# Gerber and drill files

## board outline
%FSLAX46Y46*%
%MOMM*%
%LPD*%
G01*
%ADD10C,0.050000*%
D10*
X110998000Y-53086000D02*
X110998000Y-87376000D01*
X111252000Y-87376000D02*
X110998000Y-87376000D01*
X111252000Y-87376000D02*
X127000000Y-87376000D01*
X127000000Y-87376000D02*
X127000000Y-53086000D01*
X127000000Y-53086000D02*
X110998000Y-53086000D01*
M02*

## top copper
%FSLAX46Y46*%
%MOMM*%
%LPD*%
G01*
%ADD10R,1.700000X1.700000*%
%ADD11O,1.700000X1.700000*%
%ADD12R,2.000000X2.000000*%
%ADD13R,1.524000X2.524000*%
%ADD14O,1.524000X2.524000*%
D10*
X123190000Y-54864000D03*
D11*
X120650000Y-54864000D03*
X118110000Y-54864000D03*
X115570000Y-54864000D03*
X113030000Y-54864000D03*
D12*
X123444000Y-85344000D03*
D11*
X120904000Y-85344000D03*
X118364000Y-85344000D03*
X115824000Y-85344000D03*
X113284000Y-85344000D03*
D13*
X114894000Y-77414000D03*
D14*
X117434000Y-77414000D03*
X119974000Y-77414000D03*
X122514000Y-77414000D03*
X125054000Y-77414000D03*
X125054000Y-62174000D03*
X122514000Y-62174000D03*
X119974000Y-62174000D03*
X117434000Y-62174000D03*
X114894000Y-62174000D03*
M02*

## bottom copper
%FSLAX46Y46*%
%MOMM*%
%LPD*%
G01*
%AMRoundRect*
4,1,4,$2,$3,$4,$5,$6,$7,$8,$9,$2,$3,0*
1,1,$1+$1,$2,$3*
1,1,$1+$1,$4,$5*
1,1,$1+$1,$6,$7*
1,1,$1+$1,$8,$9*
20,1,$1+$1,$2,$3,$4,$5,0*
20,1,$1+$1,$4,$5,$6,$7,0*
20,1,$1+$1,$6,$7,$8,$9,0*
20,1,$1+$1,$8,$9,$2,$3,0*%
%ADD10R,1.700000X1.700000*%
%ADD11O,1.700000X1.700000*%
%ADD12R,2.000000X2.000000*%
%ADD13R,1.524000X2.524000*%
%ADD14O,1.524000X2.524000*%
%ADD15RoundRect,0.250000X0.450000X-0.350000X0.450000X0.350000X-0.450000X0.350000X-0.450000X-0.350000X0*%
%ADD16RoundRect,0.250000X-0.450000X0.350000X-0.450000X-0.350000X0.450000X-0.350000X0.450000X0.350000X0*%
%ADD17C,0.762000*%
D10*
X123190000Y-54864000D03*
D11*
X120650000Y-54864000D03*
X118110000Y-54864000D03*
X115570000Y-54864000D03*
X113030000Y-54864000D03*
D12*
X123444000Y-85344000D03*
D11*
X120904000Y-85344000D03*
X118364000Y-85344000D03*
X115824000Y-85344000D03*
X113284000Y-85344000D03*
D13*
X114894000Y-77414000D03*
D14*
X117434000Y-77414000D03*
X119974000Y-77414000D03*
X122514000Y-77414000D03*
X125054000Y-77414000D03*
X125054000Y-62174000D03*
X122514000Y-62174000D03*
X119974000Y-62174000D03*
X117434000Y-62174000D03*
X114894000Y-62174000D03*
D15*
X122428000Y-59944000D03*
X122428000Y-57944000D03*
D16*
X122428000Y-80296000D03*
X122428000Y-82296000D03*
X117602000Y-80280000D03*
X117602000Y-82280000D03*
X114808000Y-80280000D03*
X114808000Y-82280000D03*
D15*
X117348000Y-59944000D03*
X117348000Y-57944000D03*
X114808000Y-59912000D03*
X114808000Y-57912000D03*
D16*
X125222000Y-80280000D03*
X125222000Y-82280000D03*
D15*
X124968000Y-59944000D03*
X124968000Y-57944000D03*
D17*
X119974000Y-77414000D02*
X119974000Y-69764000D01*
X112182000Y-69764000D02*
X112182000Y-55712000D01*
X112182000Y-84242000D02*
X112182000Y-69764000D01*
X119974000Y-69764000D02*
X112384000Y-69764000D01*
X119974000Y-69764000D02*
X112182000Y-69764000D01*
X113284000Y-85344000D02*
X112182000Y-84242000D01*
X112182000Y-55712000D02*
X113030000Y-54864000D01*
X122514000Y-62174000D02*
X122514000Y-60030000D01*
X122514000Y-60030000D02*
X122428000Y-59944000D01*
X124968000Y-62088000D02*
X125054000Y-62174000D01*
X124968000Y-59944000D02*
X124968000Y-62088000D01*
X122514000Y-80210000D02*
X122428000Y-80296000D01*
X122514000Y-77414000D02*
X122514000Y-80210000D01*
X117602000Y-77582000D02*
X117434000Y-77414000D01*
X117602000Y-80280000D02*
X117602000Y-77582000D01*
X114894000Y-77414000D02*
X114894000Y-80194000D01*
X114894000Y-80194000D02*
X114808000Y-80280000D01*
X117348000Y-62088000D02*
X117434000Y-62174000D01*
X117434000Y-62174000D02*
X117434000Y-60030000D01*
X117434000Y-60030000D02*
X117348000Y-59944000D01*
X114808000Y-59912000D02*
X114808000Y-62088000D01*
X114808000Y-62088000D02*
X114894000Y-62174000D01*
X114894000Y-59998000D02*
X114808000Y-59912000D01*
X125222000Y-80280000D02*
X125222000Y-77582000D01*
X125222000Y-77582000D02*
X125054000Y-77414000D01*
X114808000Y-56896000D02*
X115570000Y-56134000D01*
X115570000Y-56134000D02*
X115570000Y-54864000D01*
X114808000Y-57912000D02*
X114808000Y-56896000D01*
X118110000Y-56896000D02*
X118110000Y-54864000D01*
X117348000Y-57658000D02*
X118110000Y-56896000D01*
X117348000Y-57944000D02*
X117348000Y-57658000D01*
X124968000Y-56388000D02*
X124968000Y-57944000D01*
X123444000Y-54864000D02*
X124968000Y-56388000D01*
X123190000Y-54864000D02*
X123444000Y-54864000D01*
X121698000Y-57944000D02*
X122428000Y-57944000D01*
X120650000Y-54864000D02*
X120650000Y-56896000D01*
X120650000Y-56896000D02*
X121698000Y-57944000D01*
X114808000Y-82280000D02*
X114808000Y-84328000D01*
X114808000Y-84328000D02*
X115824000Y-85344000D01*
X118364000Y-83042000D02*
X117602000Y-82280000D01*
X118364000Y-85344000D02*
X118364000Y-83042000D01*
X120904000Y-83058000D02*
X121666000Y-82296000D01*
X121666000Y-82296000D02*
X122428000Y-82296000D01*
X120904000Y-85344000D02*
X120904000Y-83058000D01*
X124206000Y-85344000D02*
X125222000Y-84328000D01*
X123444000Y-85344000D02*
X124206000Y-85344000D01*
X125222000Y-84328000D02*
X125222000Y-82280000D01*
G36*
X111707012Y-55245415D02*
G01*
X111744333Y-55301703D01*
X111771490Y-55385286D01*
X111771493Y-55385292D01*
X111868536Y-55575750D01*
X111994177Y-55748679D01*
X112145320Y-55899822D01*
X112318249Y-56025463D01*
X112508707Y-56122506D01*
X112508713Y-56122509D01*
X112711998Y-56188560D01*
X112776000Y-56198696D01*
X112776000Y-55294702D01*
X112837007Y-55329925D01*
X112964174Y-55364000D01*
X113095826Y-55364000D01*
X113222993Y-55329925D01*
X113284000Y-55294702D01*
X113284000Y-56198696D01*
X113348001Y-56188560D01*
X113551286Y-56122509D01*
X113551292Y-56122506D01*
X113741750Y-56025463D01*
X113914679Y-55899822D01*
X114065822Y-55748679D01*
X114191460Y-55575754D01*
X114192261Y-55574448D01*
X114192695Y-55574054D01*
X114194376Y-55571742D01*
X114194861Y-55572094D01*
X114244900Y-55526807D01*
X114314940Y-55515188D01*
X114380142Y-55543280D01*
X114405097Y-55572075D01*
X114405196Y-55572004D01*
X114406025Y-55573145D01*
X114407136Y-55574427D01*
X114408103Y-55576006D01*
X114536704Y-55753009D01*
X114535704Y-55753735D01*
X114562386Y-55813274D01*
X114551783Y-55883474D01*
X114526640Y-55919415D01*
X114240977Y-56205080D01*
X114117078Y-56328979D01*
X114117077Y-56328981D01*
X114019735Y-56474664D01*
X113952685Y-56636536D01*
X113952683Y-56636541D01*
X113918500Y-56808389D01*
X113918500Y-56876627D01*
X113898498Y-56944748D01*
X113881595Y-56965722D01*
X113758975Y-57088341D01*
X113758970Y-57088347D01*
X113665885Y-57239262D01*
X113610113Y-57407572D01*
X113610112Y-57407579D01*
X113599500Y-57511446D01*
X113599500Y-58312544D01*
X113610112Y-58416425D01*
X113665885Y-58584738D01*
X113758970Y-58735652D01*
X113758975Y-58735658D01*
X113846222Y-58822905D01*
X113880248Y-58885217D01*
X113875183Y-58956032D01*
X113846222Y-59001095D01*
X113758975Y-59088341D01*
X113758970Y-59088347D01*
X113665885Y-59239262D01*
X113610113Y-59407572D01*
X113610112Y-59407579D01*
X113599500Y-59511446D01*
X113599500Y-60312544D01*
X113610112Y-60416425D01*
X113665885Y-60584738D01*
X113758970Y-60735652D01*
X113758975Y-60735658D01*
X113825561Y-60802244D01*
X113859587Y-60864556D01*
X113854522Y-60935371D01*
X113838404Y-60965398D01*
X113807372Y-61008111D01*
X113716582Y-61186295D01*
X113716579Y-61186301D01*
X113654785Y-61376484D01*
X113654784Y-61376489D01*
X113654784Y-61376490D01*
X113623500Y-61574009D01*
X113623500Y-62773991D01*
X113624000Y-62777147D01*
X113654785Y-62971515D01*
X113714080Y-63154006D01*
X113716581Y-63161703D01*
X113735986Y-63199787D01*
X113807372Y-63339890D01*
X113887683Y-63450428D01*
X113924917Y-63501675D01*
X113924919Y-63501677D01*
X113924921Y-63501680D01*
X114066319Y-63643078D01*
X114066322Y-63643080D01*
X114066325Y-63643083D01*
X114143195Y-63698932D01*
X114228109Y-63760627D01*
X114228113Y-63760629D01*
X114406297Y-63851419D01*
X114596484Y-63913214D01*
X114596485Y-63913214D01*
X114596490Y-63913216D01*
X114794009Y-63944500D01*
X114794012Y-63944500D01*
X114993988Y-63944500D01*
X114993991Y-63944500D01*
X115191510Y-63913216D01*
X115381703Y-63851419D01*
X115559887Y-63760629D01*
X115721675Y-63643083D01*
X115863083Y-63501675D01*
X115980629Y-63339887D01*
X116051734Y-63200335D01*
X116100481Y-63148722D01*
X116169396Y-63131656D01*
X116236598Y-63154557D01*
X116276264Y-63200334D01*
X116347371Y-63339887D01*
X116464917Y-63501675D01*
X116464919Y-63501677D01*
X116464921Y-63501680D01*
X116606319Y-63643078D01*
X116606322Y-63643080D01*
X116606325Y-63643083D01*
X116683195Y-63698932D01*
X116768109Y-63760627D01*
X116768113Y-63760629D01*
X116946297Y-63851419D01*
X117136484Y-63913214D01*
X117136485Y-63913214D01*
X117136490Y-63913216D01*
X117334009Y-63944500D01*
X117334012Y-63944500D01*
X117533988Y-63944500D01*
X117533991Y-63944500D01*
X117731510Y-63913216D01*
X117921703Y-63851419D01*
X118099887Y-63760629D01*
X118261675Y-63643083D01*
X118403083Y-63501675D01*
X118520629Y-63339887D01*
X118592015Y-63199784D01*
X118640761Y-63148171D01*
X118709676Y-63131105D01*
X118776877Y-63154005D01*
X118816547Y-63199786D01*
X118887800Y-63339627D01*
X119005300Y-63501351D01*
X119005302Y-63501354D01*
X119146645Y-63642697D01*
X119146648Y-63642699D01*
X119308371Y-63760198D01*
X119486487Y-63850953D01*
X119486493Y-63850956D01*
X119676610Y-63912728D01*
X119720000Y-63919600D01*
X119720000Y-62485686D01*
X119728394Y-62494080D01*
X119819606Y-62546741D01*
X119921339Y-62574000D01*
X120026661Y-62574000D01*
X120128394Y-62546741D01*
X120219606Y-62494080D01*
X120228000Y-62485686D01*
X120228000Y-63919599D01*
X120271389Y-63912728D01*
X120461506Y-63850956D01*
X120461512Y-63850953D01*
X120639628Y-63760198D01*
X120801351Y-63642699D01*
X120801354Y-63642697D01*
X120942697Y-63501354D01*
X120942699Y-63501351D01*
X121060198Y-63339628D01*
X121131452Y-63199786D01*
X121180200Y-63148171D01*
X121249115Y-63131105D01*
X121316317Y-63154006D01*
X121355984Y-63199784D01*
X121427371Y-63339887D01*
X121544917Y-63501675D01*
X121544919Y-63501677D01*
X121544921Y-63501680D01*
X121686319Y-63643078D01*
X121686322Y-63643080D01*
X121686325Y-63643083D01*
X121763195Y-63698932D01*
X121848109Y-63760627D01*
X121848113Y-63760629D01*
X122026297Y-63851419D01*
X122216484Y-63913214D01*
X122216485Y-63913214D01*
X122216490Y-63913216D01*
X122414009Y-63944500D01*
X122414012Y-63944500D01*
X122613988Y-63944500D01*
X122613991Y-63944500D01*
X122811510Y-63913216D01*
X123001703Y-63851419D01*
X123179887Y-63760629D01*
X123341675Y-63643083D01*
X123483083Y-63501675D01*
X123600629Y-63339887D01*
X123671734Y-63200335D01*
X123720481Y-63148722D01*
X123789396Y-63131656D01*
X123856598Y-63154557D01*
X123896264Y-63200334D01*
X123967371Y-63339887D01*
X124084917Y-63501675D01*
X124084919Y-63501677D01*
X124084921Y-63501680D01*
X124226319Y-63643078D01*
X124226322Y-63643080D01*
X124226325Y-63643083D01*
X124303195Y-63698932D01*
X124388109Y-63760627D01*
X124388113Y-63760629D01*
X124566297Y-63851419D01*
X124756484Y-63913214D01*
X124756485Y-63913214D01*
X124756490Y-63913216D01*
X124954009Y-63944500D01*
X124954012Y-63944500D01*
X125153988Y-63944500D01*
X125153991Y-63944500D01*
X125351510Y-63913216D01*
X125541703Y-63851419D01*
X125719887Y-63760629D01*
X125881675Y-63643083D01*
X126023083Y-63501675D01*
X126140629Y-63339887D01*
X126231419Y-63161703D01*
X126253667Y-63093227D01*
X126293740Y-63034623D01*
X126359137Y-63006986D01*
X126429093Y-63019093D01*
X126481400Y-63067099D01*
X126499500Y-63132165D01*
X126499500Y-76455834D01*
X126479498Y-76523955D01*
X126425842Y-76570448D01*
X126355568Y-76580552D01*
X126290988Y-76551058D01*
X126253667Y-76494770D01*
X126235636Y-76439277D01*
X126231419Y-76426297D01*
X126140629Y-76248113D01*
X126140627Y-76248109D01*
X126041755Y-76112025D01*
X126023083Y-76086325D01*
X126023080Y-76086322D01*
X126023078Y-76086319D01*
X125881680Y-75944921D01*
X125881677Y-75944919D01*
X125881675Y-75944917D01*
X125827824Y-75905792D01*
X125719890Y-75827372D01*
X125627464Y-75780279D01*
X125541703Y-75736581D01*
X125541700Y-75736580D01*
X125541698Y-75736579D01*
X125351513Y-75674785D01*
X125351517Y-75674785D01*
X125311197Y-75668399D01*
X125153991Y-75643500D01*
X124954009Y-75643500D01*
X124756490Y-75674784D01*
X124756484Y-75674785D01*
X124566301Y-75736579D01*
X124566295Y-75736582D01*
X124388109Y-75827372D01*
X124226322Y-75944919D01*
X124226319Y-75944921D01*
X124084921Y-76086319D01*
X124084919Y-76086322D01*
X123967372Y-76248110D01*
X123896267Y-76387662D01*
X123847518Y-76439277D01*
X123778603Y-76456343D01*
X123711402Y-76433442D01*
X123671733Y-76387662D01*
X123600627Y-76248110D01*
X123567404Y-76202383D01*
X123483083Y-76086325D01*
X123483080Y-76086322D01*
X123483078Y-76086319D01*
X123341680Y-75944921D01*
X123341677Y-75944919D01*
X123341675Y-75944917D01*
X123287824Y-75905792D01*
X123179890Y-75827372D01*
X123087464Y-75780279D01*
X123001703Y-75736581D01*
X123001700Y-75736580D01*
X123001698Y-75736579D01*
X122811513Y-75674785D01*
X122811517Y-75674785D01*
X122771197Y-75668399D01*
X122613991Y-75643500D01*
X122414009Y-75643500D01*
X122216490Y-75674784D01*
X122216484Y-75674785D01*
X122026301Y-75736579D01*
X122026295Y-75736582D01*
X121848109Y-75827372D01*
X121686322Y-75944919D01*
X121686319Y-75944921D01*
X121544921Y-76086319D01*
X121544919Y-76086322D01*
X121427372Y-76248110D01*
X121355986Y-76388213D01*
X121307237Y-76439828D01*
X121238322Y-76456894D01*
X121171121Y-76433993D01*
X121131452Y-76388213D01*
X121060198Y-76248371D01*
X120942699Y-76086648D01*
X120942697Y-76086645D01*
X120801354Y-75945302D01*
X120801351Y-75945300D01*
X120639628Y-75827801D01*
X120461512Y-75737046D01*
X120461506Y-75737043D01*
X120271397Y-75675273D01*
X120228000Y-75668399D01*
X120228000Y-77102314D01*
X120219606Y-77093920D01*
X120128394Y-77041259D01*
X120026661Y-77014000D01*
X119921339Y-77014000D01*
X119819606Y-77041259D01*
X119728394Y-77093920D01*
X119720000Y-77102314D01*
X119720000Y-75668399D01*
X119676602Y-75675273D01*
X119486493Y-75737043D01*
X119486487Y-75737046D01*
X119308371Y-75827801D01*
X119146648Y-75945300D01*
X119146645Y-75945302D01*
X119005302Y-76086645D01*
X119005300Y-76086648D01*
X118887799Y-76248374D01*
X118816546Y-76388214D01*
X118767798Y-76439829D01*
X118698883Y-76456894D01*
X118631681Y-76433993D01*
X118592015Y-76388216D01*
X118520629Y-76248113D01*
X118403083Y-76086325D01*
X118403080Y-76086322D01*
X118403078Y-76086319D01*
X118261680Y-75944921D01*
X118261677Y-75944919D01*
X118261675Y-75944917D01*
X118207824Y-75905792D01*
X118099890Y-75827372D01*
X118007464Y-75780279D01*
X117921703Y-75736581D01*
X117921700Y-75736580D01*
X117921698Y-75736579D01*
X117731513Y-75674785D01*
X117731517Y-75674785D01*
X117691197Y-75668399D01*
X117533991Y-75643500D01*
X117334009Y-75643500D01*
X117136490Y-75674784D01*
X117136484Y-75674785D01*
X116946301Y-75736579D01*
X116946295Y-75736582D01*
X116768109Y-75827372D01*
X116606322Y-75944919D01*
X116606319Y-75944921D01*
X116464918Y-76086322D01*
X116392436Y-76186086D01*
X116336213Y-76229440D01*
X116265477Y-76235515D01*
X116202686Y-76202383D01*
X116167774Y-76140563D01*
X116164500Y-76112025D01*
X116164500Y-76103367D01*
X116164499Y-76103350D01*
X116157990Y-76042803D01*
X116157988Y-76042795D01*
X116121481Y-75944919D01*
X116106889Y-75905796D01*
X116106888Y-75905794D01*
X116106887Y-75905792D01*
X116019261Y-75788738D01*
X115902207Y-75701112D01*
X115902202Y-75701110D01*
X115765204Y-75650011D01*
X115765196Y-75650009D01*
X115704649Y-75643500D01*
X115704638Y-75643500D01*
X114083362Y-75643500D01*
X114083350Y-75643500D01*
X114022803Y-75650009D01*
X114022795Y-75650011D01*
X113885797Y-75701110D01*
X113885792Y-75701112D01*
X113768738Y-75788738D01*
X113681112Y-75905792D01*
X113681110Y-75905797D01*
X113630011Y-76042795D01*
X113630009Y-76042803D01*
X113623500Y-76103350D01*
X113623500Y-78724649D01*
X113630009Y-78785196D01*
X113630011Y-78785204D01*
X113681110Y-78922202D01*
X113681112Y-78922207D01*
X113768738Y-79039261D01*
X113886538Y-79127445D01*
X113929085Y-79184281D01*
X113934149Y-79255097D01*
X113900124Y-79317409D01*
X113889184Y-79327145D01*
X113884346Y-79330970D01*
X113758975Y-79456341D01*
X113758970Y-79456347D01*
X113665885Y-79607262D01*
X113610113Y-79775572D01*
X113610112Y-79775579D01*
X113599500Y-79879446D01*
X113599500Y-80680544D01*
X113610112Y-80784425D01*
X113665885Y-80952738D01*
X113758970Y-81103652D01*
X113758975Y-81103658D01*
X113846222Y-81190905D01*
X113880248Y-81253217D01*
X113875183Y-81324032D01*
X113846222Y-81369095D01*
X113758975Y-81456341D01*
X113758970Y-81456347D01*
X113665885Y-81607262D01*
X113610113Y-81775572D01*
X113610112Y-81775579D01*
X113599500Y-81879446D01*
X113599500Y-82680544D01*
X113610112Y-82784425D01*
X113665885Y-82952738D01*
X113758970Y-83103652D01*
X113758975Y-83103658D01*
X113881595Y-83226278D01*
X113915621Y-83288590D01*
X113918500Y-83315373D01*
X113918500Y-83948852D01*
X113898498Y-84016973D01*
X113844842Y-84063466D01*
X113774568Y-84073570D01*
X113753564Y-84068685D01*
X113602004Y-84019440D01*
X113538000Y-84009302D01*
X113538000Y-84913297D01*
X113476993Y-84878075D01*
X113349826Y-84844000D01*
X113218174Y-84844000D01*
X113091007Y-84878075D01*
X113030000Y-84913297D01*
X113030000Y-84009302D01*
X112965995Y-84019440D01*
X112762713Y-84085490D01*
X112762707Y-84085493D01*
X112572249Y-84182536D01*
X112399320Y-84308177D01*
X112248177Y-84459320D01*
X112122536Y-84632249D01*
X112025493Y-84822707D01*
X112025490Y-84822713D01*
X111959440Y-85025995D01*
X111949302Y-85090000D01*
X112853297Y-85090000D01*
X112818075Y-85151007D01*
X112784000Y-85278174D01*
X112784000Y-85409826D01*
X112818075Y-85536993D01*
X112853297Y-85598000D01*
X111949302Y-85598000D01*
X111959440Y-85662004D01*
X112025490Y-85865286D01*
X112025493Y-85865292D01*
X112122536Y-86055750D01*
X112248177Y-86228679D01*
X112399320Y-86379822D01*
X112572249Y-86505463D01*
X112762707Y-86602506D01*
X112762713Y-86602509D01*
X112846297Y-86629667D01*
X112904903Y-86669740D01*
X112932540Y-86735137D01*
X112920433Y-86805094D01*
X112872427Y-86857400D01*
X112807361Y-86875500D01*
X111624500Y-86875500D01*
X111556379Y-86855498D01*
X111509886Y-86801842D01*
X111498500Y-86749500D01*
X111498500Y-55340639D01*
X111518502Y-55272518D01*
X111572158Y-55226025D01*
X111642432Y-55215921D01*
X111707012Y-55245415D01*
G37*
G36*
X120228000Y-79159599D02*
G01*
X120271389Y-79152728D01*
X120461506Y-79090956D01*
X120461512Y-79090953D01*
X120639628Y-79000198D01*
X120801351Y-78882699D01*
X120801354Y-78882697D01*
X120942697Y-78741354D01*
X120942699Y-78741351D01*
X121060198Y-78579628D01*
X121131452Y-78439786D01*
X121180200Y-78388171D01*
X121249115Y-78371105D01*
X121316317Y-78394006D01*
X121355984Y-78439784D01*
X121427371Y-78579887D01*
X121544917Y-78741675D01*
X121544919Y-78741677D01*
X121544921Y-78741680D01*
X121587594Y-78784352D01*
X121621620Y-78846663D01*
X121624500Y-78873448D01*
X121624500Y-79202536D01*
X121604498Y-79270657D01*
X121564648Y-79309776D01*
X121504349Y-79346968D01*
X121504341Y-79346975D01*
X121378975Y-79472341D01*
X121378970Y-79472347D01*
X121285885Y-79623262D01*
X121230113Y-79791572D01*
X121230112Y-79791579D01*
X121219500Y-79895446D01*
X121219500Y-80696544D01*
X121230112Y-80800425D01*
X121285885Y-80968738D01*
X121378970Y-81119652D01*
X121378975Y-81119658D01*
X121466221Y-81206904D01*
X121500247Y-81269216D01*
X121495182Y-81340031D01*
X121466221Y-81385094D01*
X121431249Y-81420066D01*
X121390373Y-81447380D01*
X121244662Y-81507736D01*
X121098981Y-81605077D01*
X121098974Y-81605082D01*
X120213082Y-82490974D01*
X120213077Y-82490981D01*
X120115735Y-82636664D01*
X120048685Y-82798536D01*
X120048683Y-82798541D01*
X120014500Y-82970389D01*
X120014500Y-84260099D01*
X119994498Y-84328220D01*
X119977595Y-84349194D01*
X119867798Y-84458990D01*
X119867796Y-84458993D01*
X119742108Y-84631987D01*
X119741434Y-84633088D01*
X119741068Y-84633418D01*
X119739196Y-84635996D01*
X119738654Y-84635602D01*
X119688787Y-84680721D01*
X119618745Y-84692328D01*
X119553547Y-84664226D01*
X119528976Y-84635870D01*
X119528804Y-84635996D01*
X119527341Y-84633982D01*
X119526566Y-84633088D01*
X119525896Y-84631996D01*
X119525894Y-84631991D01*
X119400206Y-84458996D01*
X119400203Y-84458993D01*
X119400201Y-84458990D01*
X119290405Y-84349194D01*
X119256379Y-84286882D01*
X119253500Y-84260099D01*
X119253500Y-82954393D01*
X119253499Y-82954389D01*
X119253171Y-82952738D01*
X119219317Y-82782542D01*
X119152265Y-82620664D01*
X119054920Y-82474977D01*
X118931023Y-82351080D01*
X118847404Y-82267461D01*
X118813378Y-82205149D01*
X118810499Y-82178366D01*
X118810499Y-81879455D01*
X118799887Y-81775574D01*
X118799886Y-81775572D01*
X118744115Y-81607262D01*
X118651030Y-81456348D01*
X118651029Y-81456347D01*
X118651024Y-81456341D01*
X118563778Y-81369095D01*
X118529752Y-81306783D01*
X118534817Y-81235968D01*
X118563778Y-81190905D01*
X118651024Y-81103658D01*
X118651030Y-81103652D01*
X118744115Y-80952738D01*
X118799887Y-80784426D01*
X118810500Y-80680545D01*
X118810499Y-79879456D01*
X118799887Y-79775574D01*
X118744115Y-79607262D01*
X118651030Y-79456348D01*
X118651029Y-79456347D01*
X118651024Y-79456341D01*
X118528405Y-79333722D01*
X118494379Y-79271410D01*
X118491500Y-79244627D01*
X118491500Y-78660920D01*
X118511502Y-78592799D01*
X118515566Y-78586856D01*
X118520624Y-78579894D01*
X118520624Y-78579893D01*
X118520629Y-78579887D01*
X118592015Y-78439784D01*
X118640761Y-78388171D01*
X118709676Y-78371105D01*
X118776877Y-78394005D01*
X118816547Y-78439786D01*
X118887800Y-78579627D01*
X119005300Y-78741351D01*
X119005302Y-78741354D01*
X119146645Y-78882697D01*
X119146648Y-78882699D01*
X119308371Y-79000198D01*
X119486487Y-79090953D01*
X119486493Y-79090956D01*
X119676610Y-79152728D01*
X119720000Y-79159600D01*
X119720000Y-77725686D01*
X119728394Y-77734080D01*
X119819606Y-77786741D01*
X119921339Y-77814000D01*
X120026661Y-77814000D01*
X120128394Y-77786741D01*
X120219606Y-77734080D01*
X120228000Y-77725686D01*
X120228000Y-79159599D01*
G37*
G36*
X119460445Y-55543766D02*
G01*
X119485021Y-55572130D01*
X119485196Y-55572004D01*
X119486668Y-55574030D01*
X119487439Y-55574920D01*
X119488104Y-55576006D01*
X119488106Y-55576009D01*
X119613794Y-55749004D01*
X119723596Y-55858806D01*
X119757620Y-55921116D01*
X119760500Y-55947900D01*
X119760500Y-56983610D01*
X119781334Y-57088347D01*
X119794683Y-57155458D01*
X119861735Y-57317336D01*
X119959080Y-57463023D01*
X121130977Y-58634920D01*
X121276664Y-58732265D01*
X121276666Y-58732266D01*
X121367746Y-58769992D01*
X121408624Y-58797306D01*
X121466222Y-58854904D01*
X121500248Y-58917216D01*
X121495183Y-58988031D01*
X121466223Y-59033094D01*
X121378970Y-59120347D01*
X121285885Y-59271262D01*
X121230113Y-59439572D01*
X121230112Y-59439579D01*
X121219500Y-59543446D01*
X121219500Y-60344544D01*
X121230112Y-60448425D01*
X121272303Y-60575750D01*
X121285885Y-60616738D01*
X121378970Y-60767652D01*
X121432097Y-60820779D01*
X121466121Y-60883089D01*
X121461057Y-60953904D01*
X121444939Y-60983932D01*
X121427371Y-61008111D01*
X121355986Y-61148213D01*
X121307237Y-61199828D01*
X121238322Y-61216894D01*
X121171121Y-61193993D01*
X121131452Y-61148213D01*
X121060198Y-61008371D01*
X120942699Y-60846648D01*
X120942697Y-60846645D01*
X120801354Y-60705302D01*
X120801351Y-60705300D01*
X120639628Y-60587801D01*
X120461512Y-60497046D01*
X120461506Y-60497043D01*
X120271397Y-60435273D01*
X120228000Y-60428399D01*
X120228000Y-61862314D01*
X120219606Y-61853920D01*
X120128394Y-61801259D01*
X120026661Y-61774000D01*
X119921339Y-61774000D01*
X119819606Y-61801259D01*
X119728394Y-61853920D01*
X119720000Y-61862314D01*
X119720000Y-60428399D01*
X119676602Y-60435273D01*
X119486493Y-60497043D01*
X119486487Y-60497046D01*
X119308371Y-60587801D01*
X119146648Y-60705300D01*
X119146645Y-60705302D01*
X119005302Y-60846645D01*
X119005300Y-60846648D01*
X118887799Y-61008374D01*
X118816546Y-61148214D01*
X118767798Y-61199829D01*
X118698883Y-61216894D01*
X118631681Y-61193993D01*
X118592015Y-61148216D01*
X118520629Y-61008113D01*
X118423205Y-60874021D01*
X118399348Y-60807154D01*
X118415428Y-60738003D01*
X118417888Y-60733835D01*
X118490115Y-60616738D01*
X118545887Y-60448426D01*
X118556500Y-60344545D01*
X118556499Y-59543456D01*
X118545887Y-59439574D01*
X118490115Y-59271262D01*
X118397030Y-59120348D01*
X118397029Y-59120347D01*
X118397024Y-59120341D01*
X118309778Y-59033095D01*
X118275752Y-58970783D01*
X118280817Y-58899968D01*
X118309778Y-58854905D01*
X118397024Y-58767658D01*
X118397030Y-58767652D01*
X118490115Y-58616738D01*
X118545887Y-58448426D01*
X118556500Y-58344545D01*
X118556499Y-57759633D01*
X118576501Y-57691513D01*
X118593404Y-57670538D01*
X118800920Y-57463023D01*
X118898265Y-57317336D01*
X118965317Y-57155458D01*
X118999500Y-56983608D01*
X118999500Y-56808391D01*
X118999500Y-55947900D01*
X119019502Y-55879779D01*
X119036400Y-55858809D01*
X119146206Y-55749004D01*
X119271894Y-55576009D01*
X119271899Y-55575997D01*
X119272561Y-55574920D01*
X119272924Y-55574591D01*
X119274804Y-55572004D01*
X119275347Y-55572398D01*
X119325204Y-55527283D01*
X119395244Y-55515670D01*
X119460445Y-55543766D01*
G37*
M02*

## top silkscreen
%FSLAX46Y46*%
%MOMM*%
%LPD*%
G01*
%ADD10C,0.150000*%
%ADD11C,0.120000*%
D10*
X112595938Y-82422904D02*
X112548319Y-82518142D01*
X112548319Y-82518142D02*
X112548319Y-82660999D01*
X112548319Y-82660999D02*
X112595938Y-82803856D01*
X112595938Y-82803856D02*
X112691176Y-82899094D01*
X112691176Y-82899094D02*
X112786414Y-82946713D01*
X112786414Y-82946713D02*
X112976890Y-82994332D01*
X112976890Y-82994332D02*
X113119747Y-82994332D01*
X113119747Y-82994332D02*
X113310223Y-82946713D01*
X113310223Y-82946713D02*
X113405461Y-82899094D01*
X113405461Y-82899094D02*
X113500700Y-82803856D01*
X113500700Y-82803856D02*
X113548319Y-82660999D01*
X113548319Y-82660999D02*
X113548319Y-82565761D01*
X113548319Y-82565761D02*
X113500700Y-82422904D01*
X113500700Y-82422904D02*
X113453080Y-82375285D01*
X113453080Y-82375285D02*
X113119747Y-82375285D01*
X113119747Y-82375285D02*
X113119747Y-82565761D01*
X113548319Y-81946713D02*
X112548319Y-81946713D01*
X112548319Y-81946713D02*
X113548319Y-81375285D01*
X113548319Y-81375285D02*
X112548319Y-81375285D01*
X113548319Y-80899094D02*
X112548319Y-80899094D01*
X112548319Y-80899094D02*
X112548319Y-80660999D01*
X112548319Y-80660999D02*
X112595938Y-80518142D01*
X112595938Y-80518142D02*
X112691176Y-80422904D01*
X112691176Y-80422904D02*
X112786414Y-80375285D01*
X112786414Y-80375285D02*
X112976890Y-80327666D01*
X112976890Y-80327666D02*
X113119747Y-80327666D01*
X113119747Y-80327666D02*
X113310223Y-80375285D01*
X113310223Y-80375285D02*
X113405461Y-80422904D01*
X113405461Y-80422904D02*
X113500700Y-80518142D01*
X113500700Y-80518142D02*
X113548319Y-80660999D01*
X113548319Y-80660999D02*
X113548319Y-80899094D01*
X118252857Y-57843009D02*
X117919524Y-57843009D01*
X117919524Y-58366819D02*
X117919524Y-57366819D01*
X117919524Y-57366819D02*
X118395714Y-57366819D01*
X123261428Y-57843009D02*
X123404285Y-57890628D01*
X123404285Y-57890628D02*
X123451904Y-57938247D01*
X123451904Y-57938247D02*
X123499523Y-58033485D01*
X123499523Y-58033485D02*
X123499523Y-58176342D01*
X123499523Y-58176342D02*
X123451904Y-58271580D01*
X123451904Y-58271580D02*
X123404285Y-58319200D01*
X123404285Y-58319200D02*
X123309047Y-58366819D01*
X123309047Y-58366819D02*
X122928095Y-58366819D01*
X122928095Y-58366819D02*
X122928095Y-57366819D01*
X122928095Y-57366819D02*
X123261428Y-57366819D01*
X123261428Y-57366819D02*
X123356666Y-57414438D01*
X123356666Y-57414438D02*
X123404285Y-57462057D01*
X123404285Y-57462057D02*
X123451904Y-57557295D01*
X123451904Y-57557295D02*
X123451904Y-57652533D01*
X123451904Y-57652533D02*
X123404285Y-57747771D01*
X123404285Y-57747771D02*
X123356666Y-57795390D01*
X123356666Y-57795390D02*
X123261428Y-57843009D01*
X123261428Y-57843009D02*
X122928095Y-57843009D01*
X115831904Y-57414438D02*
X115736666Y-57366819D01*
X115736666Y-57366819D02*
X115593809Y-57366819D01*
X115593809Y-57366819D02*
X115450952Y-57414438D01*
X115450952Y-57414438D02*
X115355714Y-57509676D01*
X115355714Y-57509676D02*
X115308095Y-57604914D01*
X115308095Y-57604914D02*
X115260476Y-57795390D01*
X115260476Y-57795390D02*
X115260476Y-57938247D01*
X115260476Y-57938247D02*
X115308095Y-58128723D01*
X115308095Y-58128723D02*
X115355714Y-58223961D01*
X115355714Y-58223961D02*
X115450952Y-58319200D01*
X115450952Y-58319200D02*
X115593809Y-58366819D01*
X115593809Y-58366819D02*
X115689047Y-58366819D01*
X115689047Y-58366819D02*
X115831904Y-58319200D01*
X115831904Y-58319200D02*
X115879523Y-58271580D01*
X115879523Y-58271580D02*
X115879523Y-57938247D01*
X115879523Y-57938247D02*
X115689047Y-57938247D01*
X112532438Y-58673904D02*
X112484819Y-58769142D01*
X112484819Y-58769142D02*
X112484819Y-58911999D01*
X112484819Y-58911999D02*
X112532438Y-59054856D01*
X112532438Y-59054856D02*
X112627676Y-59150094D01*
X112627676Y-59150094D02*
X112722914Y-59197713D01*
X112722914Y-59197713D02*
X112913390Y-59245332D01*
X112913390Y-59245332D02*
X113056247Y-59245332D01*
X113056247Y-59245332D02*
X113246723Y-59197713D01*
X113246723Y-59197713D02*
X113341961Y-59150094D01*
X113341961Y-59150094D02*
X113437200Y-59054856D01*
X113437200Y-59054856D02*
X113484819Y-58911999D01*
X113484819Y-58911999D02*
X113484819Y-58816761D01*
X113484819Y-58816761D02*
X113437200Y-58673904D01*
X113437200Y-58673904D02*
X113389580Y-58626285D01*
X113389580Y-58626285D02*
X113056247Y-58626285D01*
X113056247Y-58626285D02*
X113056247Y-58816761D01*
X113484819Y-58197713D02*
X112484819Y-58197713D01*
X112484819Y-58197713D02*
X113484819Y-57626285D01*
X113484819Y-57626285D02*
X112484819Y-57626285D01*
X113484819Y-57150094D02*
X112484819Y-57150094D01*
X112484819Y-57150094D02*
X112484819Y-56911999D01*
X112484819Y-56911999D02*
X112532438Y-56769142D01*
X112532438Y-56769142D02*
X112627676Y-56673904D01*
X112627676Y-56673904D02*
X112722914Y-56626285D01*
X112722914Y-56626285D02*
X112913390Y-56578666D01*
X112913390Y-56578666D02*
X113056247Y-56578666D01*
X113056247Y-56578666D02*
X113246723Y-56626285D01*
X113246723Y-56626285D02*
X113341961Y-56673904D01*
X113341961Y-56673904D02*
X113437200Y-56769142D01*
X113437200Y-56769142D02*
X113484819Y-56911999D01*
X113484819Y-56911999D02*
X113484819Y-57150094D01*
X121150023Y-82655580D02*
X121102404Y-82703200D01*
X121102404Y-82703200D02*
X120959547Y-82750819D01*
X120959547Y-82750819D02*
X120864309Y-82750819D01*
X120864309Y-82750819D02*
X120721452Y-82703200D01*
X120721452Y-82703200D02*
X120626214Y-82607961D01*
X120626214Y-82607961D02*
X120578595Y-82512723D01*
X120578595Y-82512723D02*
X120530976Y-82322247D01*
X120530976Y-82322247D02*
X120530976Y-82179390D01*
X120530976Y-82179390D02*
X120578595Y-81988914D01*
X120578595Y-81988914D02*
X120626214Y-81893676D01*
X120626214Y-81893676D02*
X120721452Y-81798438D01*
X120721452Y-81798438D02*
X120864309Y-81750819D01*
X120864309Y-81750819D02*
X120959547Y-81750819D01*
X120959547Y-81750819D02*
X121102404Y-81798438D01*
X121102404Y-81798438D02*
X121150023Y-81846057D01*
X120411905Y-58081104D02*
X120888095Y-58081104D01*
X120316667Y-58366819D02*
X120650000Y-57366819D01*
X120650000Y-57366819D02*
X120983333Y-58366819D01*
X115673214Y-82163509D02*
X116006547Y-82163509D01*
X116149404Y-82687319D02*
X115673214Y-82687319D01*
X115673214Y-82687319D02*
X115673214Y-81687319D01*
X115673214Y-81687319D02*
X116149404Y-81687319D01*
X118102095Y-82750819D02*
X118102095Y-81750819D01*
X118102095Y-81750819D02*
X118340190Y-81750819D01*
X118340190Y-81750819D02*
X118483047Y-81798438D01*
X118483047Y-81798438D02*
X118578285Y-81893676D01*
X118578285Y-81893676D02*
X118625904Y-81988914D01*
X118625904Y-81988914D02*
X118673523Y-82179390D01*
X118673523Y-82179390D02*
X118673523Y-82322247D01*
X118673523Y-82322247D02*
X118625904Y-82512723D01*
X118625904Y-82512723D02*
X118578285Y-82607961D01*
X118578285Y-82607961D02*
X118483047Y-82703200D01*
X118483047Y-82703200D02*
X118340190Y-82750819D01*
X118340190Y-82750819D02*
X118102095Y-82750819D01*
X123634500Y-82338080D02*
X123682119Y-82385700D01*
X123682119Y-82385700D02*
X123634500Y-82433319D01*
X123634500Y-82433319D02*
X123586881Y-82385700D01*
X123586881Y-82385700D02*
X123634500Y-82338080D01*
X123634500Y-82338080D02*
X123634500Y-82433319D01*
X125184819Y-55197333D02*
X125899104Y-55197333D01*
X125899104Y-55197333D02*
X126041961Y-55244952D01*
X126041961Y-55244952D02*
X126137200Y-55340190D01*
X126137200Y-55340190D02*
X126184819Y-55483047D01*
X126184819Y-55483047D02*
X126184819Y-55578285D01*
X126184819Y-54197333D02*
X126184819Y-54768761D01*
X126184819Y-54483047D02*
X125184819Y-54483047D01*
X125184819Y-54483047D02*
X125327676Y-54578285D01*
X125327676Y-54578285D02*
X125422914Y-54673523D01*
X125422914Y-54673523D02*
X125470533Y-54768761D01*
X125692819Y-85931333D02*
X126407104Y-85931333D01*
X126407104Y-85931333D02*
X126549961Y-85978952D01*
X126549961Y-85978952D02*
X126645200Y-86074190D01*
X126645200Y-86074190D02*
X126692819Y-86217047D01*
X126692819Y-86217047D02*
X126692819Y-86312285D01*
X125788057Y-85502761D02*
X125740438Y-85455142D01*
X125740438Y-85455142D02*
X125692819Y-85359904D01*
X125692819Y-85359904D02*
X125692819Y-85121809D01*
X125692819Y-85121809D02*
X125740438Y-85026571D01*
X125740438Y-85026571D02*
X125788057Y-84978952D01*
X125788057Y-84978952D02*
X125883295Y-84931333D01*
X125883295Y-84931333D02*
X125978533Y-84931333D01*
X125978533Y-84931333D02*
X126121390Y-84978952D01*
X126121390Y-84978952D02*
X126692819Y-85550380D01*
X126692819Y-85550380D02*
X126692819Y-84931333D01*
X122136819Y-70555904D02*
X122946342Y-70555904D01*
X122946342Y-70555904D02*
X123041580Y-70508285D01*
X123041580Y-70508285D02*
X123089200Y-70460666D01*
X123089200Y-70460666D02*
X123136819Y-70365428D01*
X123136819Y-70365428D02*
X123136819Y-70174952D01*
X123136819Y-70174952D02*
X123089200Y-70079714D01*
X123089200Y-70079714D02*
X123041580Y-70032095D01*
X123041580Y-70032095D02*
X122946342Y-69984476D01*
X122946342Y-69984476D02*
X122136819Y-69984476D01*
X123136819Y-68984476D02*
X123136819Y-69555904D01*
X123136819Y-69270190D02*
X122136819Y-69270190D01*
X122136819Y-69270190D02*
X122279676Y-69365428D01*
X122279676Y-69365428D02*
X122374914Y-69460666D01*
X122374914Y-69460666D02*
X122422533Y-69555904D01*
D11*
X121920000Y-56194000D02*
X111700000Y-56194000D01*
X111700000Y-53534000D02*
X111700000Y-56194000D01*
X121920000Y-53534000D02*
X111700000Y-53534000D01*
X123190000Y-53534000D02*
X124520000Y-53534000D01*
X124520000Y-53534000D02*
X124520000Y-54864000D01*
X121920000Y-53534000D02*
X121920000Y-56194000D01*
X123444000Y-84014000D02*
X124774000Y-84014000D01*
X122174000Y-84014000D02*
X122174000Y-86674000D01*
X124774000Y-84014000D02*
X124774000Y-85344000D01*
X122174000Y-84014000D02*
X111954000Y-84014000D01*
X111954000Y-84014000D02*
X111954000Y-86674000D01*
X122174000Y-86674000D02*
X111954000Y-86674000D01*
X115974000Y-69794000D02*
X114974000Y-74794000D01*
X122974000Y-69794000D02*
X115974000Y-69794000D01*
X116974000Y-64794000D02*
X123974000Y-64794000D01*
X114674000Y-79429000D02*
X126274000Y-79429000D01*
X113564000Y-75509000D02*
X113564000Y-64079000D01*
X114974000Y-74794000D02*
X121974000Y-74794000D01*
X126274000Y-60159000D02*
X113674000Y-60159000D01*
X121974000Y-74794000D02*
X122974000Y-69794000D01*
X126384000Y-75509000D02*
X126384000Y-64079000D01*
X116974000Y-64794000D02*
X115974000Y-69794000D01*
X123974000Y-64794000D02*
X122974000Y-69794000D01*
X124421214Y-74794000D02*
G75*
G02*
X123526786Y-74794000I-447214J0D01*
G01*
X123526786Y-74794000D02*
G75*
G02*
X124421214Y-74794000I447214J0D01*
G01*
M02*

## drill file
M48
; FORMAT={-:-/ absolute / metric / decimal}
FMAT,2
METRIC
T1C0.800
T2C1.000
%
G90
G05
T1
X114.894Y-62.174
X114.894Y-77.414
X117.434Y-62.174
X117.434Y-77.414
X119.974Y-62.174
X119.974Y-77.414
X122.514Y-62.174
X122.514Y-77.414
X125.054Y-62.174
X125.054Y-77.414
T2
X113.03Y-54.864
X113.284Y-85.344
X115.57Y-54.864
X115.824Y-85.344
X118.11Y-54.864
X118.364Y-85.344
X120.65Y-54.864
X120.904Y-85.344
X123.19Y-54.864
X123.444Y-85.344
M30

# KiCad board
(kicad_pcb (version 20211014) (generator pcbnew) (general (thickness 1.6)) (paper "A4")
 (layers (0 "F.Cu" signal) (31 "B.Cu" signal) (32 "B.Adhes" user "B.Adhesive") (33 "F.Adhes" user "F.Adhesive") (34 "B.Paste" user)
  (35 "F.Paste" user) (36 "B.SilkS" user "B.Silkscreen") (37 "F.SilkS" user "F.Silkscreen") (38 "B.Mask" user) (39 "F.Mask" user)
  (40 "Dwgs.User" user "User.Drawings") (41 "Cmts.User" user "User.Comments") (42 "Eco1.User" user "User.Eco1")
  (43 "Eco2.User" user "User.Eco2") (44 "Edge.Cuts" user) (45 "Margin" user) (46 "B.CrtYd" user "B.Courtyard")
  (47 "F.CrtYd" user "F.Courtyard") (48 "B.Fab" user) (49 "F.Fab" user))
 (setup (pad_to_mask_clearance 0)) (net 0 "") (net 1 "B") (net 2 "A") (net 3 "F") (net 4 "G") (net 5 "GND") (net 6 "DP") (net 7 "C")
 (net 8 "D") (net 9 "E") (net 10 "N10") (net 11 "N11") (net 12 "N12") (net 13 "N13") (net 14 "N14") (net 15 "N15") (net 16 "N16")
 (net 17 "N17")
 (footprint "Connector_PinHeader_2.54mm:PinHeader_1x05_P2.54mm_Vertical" (layer "F.Cu") (at 123.19 54.864 -90)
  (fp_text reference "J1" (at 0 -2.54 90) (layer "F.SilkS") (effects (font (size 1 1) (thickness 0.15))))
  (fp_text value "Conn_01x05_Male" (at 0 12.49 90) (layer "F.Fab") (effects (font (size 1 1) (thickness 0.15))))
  (fp_line (start 1.33 1.27) (end 1.33 11.49) (layer "F.SilkS") (width 0.12))
  (fp_line (start -1.33 11.49) (end 1.33 11.49) (layer "F.SilkS") (width 0.12))
  (fp_line (start -1.33 1.27) (end -1.33 11.49) (layer "F.SilkS") (width 0.12))
  (fp_line (start -1.33 0) (end -1.33 -1.33) (layer "F.SilkS") (width 0.12))
  (fp_line (start -1.33 -1.33) (end 0 -1.33) (layer "F.SilkS") (width 0.12))
  (fp_line (start -1.33 1.27) (end 1.33 1.27) (layer "F.SilkS") (width 0.12))
  (pad "1" thru_hole rect locked (at 0 0 270) (size 1.7 1.7) (drill 1) (layers *.Cu *.Mask) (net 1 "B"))
  (pad "2" thru_hole oval locked (at 0 2.54 270) (size 1.7 1.7) (drill 1) (layers *.Cu *.Mask) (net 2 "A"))
  (pad "3" thru_hole oval locked (at 0 5.08 270) (size 1.7 1.7) (drill 1) (layers *.Cu *.Mask) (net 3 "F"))
  (pad "4" thru_hole oval locked (at 0 7.62 270) (size 1.7 1.7) (drill 1) (layers *.Cu *.Mask) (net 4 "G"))
  (pad "5" thru_hole oval locked (at 0 10.16 270) (size 1.7 1.7) (drill 1) (layers *.Cu *.Mask) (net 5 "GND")))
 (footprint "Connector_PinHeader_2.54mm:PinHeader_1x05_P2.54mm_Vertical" (layer "F.Cu") (at 123.444 85.344 -90)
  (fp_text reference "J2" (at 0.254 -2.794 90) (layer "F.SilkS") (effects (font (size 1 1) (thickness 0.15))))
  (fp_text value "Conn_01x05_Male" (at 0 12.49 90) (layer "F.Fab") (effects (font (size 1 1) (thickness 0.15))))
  (fp_line (start -1.33 0) (end -1.33 -1.33) (layer "F.SilkS") (width 0.12))
  (fp_line (start -1.33 1.27) (end 1.33 1.27) (layer "F.SilkS") (width 0.12))
  (fp_line (start -1.33 -1.33) (end 0 -1.33) (layer "F.SilkS") (width 0.12))
  (fp_line (start -1.33 1.27) (end -1.33 11.49) (layer "F.SilkS") (width 0.12))
  (fp_line (start -1.33 11.49) (end 1.33 11.49) (layer "F.SilkS") (width 0.12))
  (fp_line (start 1.33 1.27) (end 1.33 11.49) (layer "F.SilkS") (width 0.12))
  (pad "1" thru_hole rect locked (at 0 0 270) (size 2 2) (drill 1) (layers *.Cu *.Mask) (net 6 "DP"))
  (pad "2" thru_hole oval locked (at 0 2.54 270) (size 1.7 1.7) (drill 1) (layers *.Cu *.Mask) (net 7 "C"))
  (pad "3" thru_hole oval locked (at 0 5.08 270) (size 1.7 1.7) (drill 1) (layers *.Cu *.Mask) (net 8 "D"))
  (pad "4" thru_hole oval locked (at 0 7.62 270) (size 1.7 1.7) (drill 1) (layers *.Cu *.Mask) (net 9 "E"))
  (pad "5" thru_hole oval locked (at 0 10.16 270) (size 1.7 1.7) (drill 1) (layers *.Cu *.Mask) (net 5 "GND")))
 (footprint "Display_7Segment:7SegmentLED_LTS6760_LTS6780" (layer "F.Cu") (at 114.894 77.414 90)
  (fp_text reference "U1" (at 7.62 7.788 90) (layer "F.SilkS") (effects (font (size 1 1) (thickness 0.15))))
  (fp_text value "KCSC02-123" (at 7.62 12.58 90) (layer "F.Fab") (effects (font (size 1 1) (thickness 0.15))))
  (fp_line (start 7.62 1.08) (end 2.62 0.08) (layer "F.SilkS") (width 0.12))
  (fp_line (start 7.62 8.08) (end 7.62 1.08) (layer "F.SilkS") (width 0.12))
  (fp_line (start 12.62 2.08) (end 12.62 9.08) (layer "F.SilkS") (width 0.12))
  (fp_line (start -2.015 -0.22) (end -2.015 11.38) (layer "F.SilkS") (width 0.12))
  (fp_line (start 1.905 -1.33) (end 13.335 -1.33) (layer "F.SilkS") (width 0.12))
  (fp_line (start 2.62 0.08) (end 2.62 7.08) (layer "F.SilkS") (width 0.12))
  (fp_line (start 17.255 11.38) (end 17.255 -1.22) (layer "F.SilkS") (width 0.12))
  (fp_line (start 2.62 7.08) (end 7.62 8.08) (layer "F.SilkS") (width 0.12))
  (fp_line (start 1.905 11.49) (end 13.335 11.49) (layer "F.SilkS") (width 0.12))
  (fp_line (start 12.62 2.08) (end 7.62 1.08) (layer "F.SilkS") (width 0.12))
  (fp_line (start 12.62 9.08) (end 7.62 8.08) (layer "F.SilkS") (width 0.12))
  (fp_circle (center 2.62 9.08) (end 3.067214 9.08) (layer "F.SilkS") (width 0.12) (fill none))
  (pad "1" thru_hole rect locked (at 0 0) (size 1.524 2.524) (drill 0.8) (layers *.Cu *.Mask) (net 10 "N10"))
  (pad "2" thru_hole oval locked (at 0 2.54) (size 1.524 2.524) (drill 0.8) (layers *.Cu *.Mask) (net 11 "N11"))
  (pad "3" thru_hole oval locked (at 0 5.08) (size 1.524 2.524) (drill 0.8) (layers *.Cu *.Mask) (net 5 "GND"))
  (pad "4" thru_hole oval locked (at 0 7.62) (size 1.524 2.524) (drill 0.8) (layers *.Cu *.Mask) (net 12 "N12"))
  (pad "5" thru_hole oval locked (at 0 10.16) (size 1.524 2.524) (drill 0.8) (layers *.Cu *.Mask) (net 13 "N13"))
  (pad "6" thru_hole oval locked (at 15.24 10.16) (size 1.524 2.524) (drill 0.8) (layers *.Cu *.Mask) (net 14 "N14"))
  (pad "7" thru_hole oval locked (at 15.24 7.62) (size 1.524 2.524) (drill 0.8) (layers *.Cu *.Mask) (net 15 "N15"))
  (pad "8" thru_hole oval locked (at 15.24 5.08) (size 1.524 2.524) (drill 0.8) (layers *.Cu *.Mask) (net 5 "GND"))
  (pad "9" thru_hole oval locked (at 15.24 2.54) (size 1.524 2.524) (drill 0.8) (layers *.Cu *.Mask) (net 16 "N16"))
  (pad "10" thru_hole oval locked (at 15.24 0) (size 1.524 2.524) (drill 0.8) (layers *.Cu *.Mask) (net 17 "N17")))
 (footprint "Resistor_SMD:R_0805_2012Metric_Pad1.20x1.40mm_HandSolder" (layer "B.Cu") (at 122.428 58.944 90)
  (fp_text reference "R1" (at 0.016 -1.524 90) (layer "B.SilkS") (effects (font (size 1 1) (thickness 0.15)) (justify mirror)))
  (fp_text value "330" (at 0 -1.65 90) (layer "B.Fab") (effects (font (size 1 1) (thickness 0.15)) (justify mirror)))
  (pad "1" smd roundrect locked (at -1 0 90) (size 1.2 1.4) (layers "B.Cu" "B.Paste" "B.Mask") (roundrect_rratio 0.208333) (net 15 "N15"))
  (pad "2" smd roundrect locked (at 1 0 90) (size 1.2 1.4) (layers "B.Cu" "B.Paste" "B.Mask") (roundrect_rratio 0.208333) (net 2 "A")))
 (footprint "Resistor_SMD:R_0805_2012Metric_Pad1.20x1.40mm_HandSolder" (layer "B.Cu") (at 122.428 81.296 -90)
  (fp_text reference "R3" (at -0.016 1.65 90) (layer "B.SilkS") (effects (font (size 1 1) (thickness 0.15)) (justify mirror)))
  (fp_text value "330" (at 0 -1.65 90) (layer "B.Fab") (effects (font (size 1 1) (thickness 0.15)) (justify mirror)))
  (pad "1" smd roundrect locked (at -1 0 270) (size 1.2 1.4) (layers "B.Cu" "B.Paste" "B.Mask") (roundrect_rratio 0.208333) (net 12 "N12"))
  (pad "2" smd roundrect locked (at 1 0 270) (size 1.2 1.4) (layers "B.Cu" "B.Paste" "B.Mask") (roundrect_rratio 0.208333) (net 7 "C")))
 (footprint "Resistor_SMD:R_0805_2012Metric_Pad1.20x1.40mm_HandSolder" (layer "B.Cu") (at 117.602 81.28 -90)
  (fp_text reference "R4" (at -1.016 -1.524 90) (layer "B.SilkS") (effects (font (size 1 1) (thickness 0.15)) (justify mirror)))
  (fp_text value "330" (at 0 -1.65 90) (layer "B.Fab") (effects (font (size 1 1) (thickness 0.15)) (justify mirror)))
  (pad "1" smd roundrect locked (at -1 0 270) (size 1.2 1.4) (layers "B.Cu" "B.Paste" "B.Mask") (roundrect_rratio 0.208333) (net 11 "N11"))
  (pad "2" smd roundrect locked (at 1 0 270) (size 1.2 1.4) (layers "B.Cu" "B.Paste" "B.Mask") (roundrect_rratio 0.208333) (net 8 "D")))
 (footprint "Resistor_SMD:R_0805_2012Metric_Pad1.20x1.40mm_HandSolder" (layer "B.Cu") (at 114.808 81.28 -90)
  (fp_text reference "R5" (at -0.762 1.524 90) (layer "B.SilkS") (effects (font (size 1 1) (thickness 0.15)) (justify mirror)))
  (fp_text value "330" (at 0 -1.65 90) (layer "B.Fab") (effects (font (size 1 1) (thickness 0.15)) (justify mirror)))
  (pad "1" smd roundrect locked (at -1 0 270) (size 1.2 1.4) (layers "B.Cu" "B.Paste" "B.Mask") (roundrect_rratio 0.208333) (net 10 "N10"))
  (pad "2" smd roundrect locked (at 1 0 270) (size 1.2 1.4) (layers "B.Cu" "B.Paste" "B.Mask") (roundrect_rratio 0.208333) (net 9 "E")))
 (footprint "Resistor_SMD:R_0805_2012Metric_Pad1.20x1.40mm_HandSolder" (layer "B.Cu") (at 117.348 58.944 90)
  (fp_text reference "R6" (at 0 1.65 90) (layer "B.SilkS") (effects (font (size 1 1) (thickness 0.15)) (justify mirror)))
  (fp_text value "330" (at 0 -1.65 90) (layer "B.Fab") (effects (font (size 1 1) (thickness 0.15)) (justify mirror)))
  (pad "1" smd roundrect locked (at -1 0 90) (size 1.2 1.4) (layers "B.Cu" "B.Paste" "B.Mask") (roundrect_rratio 0.208333) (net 16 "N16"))
  (pad "2" smd roundrect locked (at 1 0 90) (size 1.2 1.4) (layers "B.Cu" "B.Paste" "B.Mask") (roundrect_rratio 0.208333) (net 3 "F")))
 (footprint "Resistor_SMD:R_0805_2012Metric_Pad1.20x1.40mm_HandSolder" (layer "B.Cu") (at 114.808 58.912 90)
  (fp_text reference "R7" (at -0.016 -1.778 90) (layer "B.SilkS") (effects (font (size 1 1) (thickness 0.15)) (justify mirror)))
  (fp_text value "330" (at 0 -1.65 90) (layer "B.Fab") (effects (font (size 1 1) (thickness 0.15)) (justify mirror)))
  (pad "1" smd roundrect locked (at -1 0 90) (size 1.2 1.4) (layers "B.Cu" "B.Paste" "B.Mask") (roundrect_rratio 0.208333) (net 17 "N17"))
  (pad "2" smd roundrect locked (at 1 0 90) (size 1.2 1.4) (layers "B.Cu" "B.Paste" "B.Mask") (roundrect_rratio 0.208333) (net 4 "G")))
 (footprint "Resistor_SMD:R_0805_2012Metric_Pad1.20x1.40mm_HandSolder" (layer "B.Cu") (at 125.222 81.28 -90)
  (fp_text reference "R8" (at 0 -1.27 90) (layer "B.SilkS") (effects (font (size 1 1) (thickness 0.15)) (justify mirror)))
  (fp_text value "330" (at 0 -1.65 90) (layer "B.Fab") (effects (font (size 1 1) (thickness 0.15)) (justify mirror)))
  (pad "1" smd roundrect locked (at -1 0 270) (size 1.2 1.4) (layers "B.Cu" "B.Paste" "B.Mask") (roundrect_rratio 0.208333) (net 13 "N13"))
  (pad "2" smd roundrect locked (at 1 0 270) (size 1.2 1.4) (layers "B.Cu" "B.Paste" "B.Mask") (roundrect_rratio 0.208333) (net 6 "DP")))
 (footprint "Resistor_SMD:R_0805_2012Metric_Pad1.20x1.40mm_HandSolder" (layer "B.Cu") (at 124.968 58.944 90)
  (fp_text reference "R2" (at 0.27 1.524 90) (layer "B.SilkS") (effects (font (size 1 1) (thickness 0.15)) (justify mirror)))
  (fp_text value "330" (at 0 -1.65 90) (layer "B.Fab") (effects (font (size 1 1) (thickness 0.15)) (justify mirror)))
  (pad "1" smd roundrect locked (at -1 0 90) (size 1.2 1.4) (layers "B.Cu" "B.Paste" "B.Mask") (roundrect_rratio 0.208333) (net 14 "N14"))
  (pad "2" smd roundrect locked (at 1 0 90) (size 1.2 1.4) (layers "B.Cu" "B.Paste" "B.Mask") (roundrect_rratio 0.208333) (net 1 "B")))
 (gr_line (start 110.998 53.086) (end 110.998 87.376) (layer "Edge.Cuts") (width 0.05))
 (gr_line (start 111.252 87.376) (end 110.998 87.376) (layer "Edge.Cuts") (width 0.05))
 (gr_line (start 111.252 87.376) (end 127 87.376) (layer "Edge.Cuts") (width 0.05))
 (gr_line (start 127 87.376) (end 127 53.086) (layer "Edge.Cuts") (width 0.05))
 (gr_line (start 127 53.086) (end 110.998 53.086) (layer "Edge.Cuts") (width 0.05))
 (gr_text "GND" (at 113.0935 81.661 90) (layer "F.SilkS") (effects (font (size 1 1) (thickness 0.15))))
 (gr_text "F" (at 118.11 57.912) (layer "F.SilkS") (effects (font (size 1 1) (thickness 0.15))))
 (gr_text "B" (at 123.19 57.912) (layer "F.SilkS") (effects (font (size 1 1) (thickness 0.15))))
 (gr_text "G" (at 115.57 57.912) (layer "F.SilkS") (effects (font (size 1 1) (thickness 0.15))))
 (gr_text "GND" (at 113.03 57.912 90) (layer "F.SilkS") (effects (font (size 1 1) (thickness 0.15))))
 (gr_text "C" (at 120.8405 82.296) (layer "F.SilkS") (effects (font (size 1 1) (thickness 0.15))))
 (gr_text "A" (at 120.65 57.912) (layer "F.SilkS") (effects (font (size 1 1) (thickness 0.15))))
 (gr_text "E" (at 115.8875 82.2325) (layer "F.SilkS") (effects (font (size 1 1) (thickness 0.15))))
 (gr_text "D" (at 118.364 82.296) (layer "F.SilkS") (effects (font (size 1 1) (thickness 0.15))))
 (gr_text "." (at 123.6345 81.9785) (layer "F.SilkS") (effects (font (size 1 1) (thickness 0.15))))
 (segment (start 119.974 77.414) (end 119.974 69.764) (width 0.762) (layer "B.Cu") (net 5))
 (segment (start 112.182 69.764) (end 112.182 55.712) (width 0.762) (layer "B.Cu") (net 5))
 (segment (start 112.182 84.242) (end 112.182 69.764) (width 0.762) (layer "B.Cu") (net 5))
 (segment (start 119.974 69.764) (end 112.384 69.764) (width 0.762) (layer "B.Cu") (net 5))
 (segment (start 119.974 69.764) (end 112.182 69.764) (width 0.762) (layer "B.Cu") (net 5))
 (segment (start 113.284 85.344) (end 112.182 84.242) (width 0.762) (layer "B.Cu") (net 5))
 (segment (start 112.182 55.712) (end 113.03 54.864) (width 0.762) (layer "B.Cu") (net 5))
 (segment (start 122.514 62.174) (end 122.514 60.03) (width 0.762) (layer "B.Cu") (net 15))
 (segment (start 122.514 60.03) (end 122.428 59.944) (width 0.762) (layer "B.Cu") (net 15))
 (segment (start 124.968 62.088) (end 125.054 62.174) (width 0.762) (layer "B.Cu") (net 14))
 (segment (start 124.968 59.944) (end 124.968 62.088) (width 0.762) (layer "B.Cu") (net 14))
 (segment (start 122.514 80.21) (end 122.428 80.296) (width 0.762) (layer "B.Cu") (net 12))
 (segment (start 122.514 77.414) (end 122.514 80.21) (width 0.762) (layer "B.Cu") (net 12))
 (segment (start 117.602 77.582) (end 117.434 77.414) (width 0.762) (layer "B.Cu") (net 11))
 (segment (start 117.602 80.28) (end 117.602 77.582) (width 0.762) (layer "B.Cu") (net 11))
 (segment (start 114.894 77.414) (end 114.894 80.194) (width 0.762) (layer "B.Cu") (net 10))
 (segment (start 114.894 80.194) (end 114.808 80.28) (width 0.762) (layer "B.Cu") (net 10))
 (segment (start 117.348 62.088) (end 117.434 62.174) (width 0.762) (layer "B.Cu") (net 16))
 (segment (start 117.434 62.174) (end 117.434 60.03) (width 0.762) (layer "B.Cu") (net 16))
 (segment (start 117.434 60.03) (end 117.348 59.944) (width 0.762) (layer "B.Cu") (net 16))
 (segment (start 114.808 59.912) (end 114.808 62.088) (width 0.762) (layer "B.Cu") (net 17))
 (segment (start 114.808 62.088) (end 114.894 62.174) (width 0.762) (layer "B.Cu") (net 17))
 (segment (start 114.894 59.998) (end 114.808 59.912) (width 0.762) (layer "B.Cu") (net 17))
 (segment (start 125.222 80.28) (end 125.222 77.582) (width 0.762) (layer "B.Cu") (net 13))
 (segment (start 125.222 77.582) (end 125.054 77.414) (width 0.762) (layer "B.Cu") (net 13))
 (segment (start 114.808 56.896) (end 115.57 56.134) (width 0.762) (layer "B.Cu") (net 4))
 (segment (start 115.57 56.134) (end 115.57 54.864) (width 0.762) (layer "B.Cu") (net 4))
 (segment (start 114.808 57.912) (end 114.808 56.896) (width 0.762) (layer "B.Cu") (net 4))
 (segment (start 118.11 56.896) (end 118.11 54.864) (width 0.762) (layer "B.Cu") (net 3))
 (segment (start 117.348 57.658) (end 118.11 56.896) (width 0.762) (layer "B.Cu") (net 3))
 (segment (start 117.348 57.944) (end 117.348 57.658) (width 0.762) (layer "B.Cu") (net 3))
 (segment (start 124.968 56.388) (end 124.968 57.944) (width 0.762) (layer "B.Cu") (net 1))
 (segment (start 123.444 54.864) (end 124.968 56.388) (width 0.762) (layer "B.Cu") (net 1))
 (segment (start 123.19 54.864) (end 123.444 54.864) (width 0.762) (layer "B.Cu") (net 1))
 (segment (start 121.698 57.944) (end 122.428 57.944) (width 0.762) (layer "B.Cu") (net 2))
 (segment (start 120.65 54.864) (end 120.65 56.896) (width 0.762) (layer "B.Cu") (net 2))
 (segment (start 120.65 56.896) (end 121.698 57.944) (width 0.762) (layer "B.Cu") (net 2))
 (segment (start 114.808 82.28) (end 114.808 84.328) (width 0.762) (layer "B.Cu") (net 9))
 (segment (start 114.808 84.328) (end 115.824 85.344) (width 0.762) (layer "B.Cu") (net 9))
 (segment (start 118.364 83.042) (end 117.602 82.28) (width 0.762) (layer "B.Cu") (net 8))
 (segment (start 118.364 85.344) (end 118.364 83.042) (width 0.762) (layer "B.Cu") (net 8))
 (segment (start 120.904 83.058) (end 121.666 82.296) (width 0.762) (layer "B.Cu") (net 7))
 (segment (start 121.666 82.296) (end 122.428 82.296) (width 0.762) (layer "B.Cu") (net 7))
 (segment (start 120.904 85.344) (end 120.904 83.058) (width 0.762) (layer "B.Cu") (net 7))
 (segment (start 124.206 85.344) (end 125.222 84.328) (width 0.762) (layer "B.Cu") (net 6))
 (segment (start 123.444 85.344) (end 124.206 85.344) (width 0.762) (layer "B.Cu") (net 6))
 (segment (start 125.222 84.328) (end 125.222 82.28) (width 0.762) (layer "B.Cu") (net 6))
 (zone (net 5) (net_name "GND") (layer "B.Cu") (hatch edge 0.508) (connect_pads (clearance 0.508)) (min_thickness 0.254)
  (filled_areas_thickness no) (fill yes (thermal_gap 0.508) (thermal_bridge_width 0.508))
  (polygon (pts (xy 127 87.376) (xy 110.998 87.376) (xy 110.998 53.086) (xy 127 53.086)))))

